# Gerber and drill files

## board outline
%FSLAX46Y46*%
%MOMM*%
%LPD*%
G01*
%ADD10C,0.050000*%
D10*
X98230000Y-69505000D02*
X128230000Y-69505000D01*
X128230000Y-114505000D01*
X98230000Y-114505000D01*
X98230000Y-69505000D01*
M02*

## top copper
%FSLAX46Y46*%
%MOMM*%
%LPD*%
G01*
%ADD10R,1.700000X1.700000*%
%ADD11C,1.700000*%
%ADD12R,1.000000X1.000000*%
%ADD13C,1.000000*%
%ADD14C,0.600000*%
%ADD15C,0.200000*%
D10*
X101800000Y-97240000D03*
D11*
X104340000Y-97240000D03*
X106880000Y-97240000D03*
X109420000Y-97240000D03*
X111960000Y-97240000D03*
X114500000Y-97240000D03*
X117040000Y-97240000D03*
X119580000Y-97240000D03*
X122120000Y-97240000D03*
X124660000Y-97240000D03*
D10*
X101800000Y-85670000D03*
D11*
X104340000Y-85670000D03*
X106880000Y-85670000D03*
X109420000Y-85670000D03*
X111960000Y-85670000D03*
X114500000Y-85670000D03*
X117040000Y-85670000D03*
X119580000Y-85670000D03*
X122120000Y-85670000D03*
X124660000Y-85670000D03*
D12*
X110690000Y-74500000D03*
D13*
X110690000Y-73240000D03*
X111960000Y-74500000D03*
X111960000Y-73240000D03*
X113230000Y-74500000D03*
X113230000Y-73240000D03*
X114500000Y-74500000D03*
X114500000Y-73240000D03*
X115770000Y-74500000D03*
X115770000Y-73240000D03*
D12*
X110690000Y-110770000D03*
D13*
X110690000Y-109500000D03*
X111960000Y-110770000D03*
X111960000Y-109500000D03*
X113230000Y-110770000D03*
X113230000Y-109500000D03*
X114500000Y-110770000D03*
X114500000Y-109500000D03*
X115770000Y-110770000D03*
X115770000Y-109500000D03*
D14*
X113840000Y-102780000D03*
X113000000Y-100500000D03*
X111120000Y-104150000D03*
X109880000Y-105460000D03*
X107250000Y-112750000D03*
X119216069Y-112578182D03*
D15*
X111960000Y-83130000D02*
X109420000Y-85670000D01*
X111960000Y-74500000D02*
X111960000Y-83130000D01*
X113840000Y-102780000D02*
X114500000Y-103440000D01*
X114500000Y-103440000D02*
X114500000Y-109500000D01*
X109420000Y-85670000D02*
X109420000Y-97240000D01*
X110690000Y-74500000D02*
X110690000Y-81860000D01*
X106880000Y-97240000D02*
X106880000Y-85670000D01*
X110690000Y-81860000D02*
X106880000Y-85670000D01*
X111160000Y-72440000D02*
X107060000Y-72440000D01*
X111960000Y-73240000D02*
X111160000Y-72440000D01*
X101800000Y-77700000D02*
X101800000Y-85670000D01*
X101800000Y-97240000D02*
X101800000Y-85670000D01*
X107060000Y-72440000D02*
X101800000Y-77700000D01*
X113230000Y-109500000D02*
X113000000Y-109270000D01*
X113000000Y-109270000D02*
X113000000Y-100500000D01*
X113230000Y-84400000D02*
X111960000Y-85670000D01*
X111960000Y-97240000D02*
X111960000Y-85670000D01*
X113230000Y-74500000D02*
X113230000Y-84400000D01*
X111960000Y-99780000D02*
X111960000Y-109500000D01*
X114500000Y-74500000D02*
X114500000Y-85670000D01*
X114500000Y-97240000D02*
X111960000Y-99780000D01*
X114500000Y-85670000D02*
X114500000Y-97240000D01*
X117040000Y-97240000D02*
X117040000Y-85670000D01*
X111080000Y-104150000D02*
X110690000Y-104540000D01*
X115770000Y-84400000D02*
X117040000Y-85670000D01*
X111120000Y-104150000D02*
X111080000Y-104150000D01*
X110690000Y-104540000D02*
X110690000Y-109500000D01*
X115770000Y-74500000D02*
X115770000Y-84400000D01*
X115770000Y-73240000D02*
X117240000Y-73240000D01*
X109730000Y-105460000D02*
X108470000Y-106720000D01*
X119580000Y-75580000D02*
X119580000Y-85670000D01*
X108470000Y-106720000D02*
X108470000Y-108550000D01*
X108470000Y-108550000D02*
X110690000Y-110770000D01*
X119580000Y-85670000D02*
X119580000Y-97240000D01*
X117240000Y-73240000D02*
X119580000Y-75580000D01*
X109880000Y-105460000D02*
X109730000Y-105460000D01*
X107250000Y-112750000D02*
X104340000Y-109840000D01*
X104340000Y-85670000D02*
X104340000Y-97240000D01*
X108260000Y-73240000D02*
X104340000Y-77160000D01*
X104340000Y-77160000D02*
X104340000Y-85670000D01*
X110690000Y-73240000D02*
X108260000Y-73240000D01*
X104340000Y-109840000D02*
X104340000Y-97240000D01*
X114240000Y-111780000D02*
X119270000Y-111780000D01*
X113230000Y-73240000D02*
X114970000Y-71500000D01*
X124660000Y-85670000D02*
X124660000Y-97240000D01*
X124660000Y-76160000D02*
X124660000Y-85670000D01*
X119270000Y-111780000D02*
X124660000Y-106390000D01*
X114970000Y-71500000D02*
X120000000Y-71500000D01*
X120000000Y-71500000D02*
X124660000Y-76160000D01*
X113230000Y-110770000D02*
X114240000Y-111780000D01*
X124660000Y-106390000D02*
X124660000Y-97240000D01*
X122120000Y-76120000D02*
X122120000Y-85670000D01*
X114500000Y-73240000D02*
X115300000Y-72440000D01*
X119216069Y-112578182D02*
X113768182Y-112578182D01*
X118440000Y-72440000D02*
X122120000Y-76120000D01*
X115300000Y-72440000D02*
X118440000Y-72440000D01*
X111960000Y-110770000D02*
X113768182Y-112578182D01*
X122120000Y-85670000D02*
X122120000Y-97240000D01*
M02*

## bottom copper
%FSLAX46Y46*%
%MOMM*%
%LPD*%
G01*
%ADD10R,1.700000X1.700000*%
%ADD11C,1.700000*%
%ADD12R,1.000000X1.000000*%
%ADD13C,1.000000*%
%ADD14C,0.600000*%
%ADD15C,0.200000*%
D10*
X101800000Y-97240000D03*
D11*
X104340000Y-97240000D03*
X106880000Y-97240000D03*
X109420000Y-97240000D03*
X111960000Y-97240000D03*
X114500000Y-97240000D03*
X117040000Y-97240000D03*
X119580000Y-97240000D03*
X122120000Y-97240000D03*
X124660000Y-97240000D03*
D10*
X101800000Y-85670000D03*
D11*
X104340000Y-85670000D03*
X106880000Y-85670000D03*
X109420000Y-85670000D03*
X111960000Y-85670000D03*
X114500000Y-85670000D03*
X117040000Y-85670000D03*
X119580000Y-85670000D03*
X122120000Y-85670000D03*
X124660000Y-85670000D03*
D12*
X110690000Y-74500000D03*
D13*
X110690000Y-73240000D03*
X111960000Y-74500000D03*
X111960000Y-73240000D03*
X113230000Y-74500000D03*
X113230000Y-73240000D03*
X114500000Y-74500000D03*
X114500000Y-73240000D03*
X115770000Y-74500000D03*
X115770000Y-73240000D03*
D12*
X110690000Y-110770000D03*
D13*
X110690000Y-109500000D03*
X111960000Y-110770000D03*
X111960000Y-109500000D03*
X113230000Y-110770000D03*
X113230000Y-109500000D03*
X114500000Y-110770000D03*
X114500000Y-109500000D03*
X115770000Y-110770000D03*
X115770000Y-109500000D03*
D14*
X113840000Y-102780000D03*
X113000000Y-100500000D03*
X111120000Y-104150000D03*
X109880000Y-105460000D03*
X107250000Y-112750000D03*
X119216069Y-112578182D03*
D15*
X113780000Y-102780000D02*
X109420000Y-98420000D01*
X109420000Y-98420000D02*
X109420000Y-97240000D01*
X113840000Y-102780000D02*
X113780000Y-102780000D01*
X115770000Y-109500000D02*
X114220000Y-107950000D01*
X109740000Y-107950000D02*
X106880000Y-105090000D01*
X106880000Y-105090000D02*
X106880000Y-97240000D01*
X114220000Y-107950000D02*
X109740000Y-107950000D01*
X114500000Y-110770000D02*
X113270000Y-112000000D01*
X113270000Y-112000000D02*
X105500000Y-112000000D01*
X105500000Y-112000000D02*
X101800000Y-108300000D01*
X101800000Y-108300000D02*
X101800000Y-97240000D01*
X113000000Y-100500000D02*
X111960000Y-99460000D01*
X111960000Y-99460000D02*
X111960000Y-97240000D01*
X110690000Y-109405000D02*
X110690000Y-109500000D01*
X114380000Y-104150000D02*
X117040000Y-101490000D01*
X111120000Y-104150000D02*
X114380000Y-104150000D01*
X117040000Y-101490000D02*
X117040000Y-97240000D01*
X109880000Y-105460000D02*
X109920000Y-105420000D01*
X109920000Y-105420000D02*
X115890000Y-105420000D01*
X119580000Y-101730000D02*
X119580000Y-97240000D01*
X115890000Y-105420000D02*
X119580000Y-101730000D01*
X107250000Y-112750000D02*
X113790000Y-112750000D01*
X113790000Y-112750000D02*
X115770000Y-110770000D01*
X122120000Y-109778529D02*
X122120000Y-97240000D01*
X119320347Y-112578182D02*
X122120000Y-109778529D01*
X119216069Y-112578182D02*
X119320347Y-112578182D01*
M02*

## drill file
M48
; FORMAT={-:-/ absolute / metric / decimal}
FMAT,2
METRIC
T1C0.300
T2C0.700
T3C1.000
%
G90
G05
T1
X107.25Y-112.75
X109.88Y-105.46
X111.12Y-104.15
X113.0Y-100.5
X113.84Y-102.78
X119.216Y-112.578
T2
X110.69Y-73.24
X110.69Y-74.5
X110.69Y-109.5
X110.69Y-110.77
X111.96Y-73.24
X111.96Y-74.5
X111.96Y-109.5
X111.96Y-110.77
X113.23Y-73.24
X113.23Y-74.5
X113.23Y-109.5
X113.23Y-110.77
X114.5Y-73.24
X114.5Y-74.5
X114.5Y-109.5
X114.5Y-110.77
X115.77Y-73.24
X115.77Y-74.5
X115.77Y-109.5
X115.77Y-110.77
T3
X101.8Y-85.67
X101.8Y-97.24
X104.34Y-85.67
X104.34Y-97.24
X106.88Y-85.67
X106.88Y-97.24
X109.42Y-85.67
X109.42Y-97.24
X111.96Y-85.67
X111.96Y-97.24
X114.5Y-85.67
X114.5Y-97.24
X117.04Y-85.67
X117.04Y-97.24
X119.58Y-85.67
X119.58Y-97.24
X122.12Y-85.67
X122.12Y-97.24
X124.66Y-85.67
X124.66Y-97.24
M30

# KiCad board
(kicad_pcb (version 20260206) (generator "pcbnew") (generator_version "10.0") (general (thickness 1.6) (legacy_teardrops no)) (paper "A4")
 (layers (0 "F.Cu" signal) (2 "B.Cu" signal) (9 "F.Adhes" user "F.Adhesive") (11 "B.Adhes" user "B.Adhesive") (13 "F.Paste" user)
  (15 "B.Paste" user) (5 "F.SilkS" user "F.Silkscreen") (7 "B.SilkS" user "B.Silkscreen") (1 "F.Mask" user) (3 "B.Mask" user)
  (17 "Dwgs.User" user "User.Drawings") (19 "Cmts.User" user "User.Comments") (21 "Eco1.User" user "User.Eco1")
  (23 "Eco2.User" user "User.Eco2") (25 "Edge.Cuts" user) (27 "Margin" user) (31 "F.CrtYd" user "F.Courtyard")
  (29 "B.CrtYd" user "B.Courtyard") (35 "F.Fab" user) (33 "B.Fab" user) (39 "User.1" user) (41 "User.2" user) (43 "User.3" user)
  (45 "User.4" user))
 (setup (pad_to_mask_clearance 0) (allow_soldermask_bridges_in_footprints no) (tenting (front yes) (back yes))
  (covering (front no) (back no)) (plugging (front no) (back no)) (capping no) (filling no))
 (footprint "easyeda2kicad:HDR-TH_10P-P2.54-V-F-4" (layer "F.Cu") (at 113.23 97.24)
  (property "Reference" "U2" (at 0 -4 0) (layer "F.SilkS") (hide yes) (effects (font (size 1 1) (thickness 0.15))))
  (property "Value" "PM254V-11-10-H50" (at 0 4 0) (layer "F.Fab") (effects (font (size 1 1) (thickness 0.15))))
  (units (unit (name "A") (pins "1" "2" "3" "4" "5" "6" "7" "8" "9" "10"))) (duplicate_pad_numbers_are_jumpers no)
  (pad "1" thru_hole rect (at -11.43 0) (size 1.7 1.7) (drill 0.999998) (layers "*.Cu" "*.Mask") (remove_unused_layers no) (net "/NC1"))
  (pad "2" thru_hole circle (at -8.89 0) (size 1.7 1.7) (drill 0.999998) (layers "*.Cu" "*.Mask") (remove_unused_layers no) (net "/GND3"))
  (pad "3" thru_hole circle (at -6.35 0) (size 1.7 1.7) (drill 0.999998) (layers "*.Cu" "*.Mask") (remove_unused_layers no) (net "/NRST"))
  (pad "4" thru_hole circle (at -3.81 0) (size 1.7 1.7) (drill 0.999998) (layers "*.Cu" "*.Mask") (remove_unused_layers no) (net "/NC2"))
  (pad "5" thru_hole circle (at -1.27 0) (size 1.7 1.7) (drill 0.999998) (layers "*.Cu" "*.Mask") (remove_unused_layers no)
   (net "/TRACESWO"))
  (pad "6" thru_hole circle (at 1.27 0) (size 1.7 1.7) (drill 0.999998) (layers "*.Cu" "*.Mask") (remove_unused_layers no) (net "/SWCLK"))
  (pad "7" thru_hole circle (at 3.81 0) (size 1.7 1.7) (drill 0.999998) (layers "*.Cu" "*.Mask") (remove_unused_layers no) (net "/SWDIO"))
  (pad "8" thru_hole circle (at 6.35 0) (size 1.7 1.7) (drill 0.999998) (layers "*.Cu" "*.Mask") (remove_unused_layers no) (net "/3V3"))
  (pad "9" thru_hole circle (at 8.89 0) (size 1.7 1.7) (drill 0.999998) (layers "*.Cu" "*.Mask") (remove_unused_layers no) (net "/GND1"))
  (pad "10" thru_hole circle (at 11.43 0) (size 1.7 1.7) (drill 0.999998) (layers "*.Cu" "*.Mask") (remove_unused_layers no) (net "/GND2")))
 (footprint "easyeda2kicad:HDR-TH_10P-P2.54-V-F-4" (layer "F.Cu") (at 113.23 85.67)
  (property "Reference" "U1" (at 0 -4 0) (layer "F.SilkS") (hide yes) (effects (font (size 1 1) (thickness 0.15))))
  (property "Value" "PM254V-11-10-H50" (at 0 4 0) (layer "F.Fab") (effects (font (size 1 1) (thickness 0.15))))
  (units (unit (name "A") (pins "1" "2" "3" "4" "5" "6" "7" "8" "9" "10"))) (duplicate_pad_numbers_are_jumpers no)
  (pad "1" thru_hole rect (at -11.43 0) (size 1.7 1.7) (drill 0.999998) (layers "*.Cu" "*.Mask") (remove_unused_layers no) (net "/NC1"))
  (pad "2" thru_hole circle (at -8.89 0) (size 1.7 1.7) (drill 0.999998) (layers "*.Cu" "*.Mask") (remove_unused_layers no) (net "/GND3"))
  (pad "3" thru_hole circle (at -6.35 0) (size 1.7 1.7) (drill 0.999998) (layers "*.Cu" "*.Mask") (remove_unused_layers no) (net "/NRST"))
  (pad "4" thru_hole circle (at -3.81 0) (size 1.7 1.7) (drill 0.999998) (layers "*.Cu" "*.Mask") (remove_unused_layers no) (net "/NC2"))
  (pad "5" thru_hole circle (at -1.27 0) (size 1.7 1.7) (drill 0.999998) (layers "*.Cu" "*.Mask") (remove_unused_layers no)
   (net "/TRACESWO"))
  (pad "6" thru_hole circle (at 1.27 0) (size 1.7 1.7) (drill 0.999998) (layers "*.Cu" "*.Mask") (remove_unused_layers no) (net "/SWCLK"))
  (pad "7" thru_hole circle (at 3.81 0) (size 1.7 1.7) (drill 0.999998) (layers "*.Cu" "*.Mask") (remove_unused_layers no) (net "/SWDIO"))
  (pad "8" thru_hole circle (at 6.35 0) (size 1.7 1.7) (drill 0.999998) (layers "*.Cu" "*.Mask") (remove_unused_layers no) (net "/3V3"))
  (pad "9" thru_hole circle (at 8.89 0) (size 1.7 1.7) (drill 0.999998) (layers "*.Cu" "*.Mask") (remove_unused_layers no) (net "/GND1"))
  (pad "10" thru_hole circle (at 11.43 0) (size 1.7 1.7) (drill 0.999998) (layers "*.Cu" "*.Mask") (remove_unused_layers no) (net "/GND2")))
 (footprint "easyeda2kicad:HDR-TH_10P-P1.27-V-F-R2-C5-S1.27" (layer "F.Cu") (at 113.23 73.87)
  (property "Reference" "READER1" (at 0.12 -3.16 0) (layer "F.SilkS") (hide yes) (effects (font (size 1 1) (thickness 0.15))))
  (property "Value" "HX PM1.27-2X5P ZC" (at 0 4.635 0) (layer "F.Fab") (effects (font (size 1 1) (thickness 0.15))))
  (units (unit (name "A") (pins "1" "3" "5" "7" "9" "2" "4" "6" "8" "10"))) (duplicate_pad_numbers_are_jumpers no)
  (pad "1" thru_hole rect (at -2.54 0.63) (size 1 1) (drill 0.700024) (layers "*.Cu" "*.Mask") (remove_unused_layers no) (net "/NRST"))
  (pad "2" thru_hole circle (at -2.54 -0.63) (size 1 1) (drill 0.700024) (layers "*.Cu" "*.Mask") (remove_unused_layers no) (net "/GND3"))
  (pad "3" thru_hole circle (at -1.27 0.63) (size 1 1) (drill 0.700024) (layers "*.Cu" "*.Mask") (remove_unused_layers no) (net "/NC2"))
  (pad "4" thru_hole circle (at -1.27 -0.63) (size 1 1) (drill 0.700024) (layers "*.Cu" "*.Mask") (remove_unused_layers no) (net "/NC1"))
  (pad "5" thru_hole circle (at 0 0.63) (size 1 1) (drill 0.700024) (layers "*.Cu" "*.Mask") (remove_unused_layers no) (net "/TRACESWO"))
  (pad "6" thru_hole circle (at 0 -0.63) (size 1 1) (drill 0.700024) (layers "*.Cu" "*.Mask") (remove_unused_layers no) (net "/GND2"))
  (pad "7" thru_hole circle (at 1.27 0.63) (size 1 1) (drill 0.700024) (layers "*.Cu" "*.Mask") (remove_unused_layers no) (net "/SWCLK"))
  (pad "8" thru_hole circle (at 1.27 -0.63) (size 1 1) (drill 0.700024) (layers "*.Cu" "*.Mask") (remove_unused_layers no) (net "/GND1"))
  (pad "9" thru_hole circle (at 2.54 0.63) (size 1 1) (drill 0.700024) (layers "*.Cu" "*.Mask") (remove_unused_layers no) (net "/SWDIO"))
  (pad "10" thru_hole circle (at 2.54 -0.63) (size 1 1) (drill 0.700024) (layers "*.Cu" "*.Mask") (remove_unused_layers no) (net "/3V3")))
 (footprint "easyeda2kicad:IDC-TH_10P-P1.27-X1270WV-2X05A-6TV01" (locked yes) (layer "F.Cu") (at 113.23 110.14)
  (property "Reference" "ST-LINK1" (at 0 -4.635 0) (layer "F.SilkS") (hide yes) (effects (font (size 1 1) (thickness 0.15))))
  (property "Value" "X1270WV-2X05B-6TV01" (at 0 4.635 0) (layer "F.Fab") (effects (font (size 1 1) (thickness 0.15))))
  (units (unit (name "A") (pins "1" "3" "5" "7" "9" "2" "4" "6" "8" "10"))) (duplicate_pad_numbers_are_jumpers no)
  (pad "1" thru_hole rect (at -2.54 0.63) (size 1 1) (drill 0.700024) (layers "*.Cu" "*.Mask") (remove_unused_layers no) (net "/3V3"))
  (pad "2" thru_hole circle (at -2.54 -0.64) (size 1 1) (drill 0.700024) (layers "*.Cu" "*.Mask") (remove_unused_layers no) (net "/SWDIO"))
  (pad "3" thru_hole circle (at -1.27 0.63) (size 1 1) (drill 0.700024) (layers "*.Cu" "*.Mask") (remove_unused_layers no) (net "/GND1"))
  (pad "4" thru_hole circle (at -1.27 -0.64) (size 1 1) (drill 0.700024) (layers "*.Cu" "*.Mask") (remove_unused_layers no) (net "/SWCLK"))
  (pad "5" thru_hole circle (at 0 0.63) (size 1 1) (drill 0.700024) (layers "*.Cu" "*.Mask") (remove_unused_layers no) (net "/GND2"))
  (pad "6" thru_hole circle (at 0 -0.64) (size 1 1) (drill 0.700024) (layers "*.Cu" "*.Mask") (remove_unused_layers no) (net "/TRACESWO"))
  (pad "7" thru_hole circle (at 1.27 0.63) (size 1 1) (drill 0.700024) (layers "*.Cu" "*.Mask") (remove_unused_layers no) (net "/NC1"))
  (pad "8" thru_hole circle (at 1.27 -0.64) (size 1 1) (drill 0.700024) (layers "*.Cu" "*.Mask") (remove_unused_layers no) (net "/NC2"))
  (pad "9" thru_hole circle (at 2.54 0.63) (size 1 1) (drill 0.700024) (layers "*.Cu" "*.Mask") (remove_unused_layers no) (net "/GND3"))
  (pad "10" thru_hole circle (at 2.54 -0.64) (size 1 1) (drill 0.700024) (layers "*.Cu" "*.Mask") (remove_unused_layers no) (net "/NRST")))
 (gr_rect (start 98.23 69.505) (end 128.23 114.505) (stroke (width 0.05) (type default)) (fill no) (layer "Edge.Cuts"))
 (segment (start 111.96 83.13) (end 109.42 85.67) (width 0.2) (layer "F.Cu") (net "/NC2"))
 (segment (start 111.96 74.5) (end 111.96 83.13) (width 0.2) (layer "F.Cu") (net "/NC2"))
 (segment (start 113.84 102.78) (end 114.5 103.44) (width 0.2) (layer "F.Cu") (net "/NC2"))
 (segment (start 114.5 103.44) (end 114.5 109.5) (width 0.2) (layer "F.Cu") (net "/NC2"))
 (segment (start 109.42 85.67) (end 109.42 97.24) (width 0.2) (layer "F.Cu") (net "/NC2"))
 (via (at 113.84 102.78) (size 0.6) (drill 0.3) (layers "F.Cu" "B.Cu") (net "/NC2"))
 (segment (start 113.78 102.78) (end 109.42 98.42) (width 0.2) (layer "B.Cu") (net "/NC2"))
 (segment (start 109.42 98.42) (end 109.42 97.24) (width 0.2) (layer "B.Cu") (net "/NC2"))
 (segment (start 113.84 102.78) (end 113.78 102.78) (width 0.2) (layer "B.Cu") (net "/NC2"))
 (segment (start 110.69 74.5) (end 110.69 81.86) (width 0.2) (layer "F.Cu") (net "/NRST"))
 (segment (start 106.88 97.24) (end 106.88 85.67) (width 0.2) (layer "F.Cu") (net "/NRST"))
 (segment (start 110.69 81.86) (end 106.88 85.67) (width 0.2) (layer "F.Cu") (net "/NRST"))
 (segment (start 115.77 109.5) (end 114.22 107.95) (width 0.2) (layer "B.Cu") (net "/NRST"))
 (segment (start 109.74 107.95) (end 106.88 105.09) (width 0.2) (layer "B.Cu") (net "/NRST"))
 (segment (start 106.88 105.09) (end 106.88 97.24) (width 0.2) (layer "B.Cu") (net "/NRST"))
 (segment (start 114.22 107.95) (end 109.74 107.95) (width 0.2) (layer "B.Cu") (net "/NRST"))
 (segment (start 111.16 72.44) (end 107.06 72.44) (width 0.2) (layer "F.Cu") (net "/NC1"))
 (segment (start 111.96 73.24) (end 111.16 72.44) (width 0.2) (layer "F.Cu") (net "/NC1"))
 (segment (start 101.8 77.7) (end 101.8 85.67) (width 0.2) (layer "F.Cu") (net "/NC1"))
 (segment (start 101.8 97.24) (end 101.8 85.67) (width 0.2) (layer "F.Cu") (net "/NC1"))
 (segment (start 107.06 72.44) (end 101.8 77.7) (width 0.2) (layer "F.Cu") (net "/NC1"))
 (segment (start 114.5 110.77) (end 113.27 112) (width 0.2) (layer "B.Cu") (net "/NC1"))
 (segment (start 113.27 112) (end 105.5 112) (width 0.2) (layer "B.Cu") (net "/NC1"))
 (segment (start 105.5 112) (end 101.8 108.3) (width 0.2) (layer "B.Cu") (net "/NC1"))
 (segment (start 101.8 108.3) (end 101.8 97.24) (width 0.2) (layer "B.Cu") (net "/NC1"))
 (segment (start 113.23 109.5) (end 113 109.27) (width 0.2) (layer "F.Cu") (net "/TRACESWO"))
 (segment (start 113 109.27) (end 113 100.5) (width 0.2) (layer "F.Cu") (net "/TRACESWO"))
 (segment (start 113.23 84.4) (end 111.96 85.67) (width 0.2) (layer "F.Cu") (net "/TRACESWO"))
 (segment (start 111.96 97.24) (end 111.96 85.67) (width 0.2) (layer "F.Cu") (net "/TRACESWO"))
 (segment (start 113.23 74.5) (end 113.23 84.4) (width 0.2) (layer "F.Cu") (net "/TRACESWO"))
 (via (at 113 100.5) (size 0.6) (drill 0.3) (layers "F.Cu" "B.Cu") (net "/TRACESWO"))
 (segment (start 113 100.5) (end 111.96 99.46) (width 0.2) (layer "B.Cu") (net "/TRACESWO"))
 (segment (start 111.96 99.46) (end 111.96 97.24) (width 0.2) (layer "B.Cu") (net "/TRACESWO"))
 (segment (start 111.96 99.78) (end 111.96 109.5) (width 0.2) (layer "F.Cu") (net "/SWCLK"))
 (segment (start 114.5 74.5) (end 114.5 85.67) (width 0.2) (layer "F.Cu") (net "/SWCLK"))
 (segment (start 114.5 97.24) (end 111.96 99.78) (width 0.2) (layer "F.Cu") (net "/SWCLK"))
 (segment (start 114.5 85.67) (end 114.5 97.24) (width 0.2) (layer "F.Cu") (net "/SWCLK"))
 (segment (start 117.04 97.24) (end 117.04 85.67) (width 0.2) (layer "F.Cu") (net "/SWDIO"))
 (segment (start 111.08 104.15) (end 110.69 104.54) (width 0.2) (layer "F.Cu") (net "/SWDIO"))
 (segment (start 115.77 84.4) (end 117.04 85.67) (width 0.2) (layer "F.Cu") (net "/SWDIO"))
 (segment (start 111.12 104.15) (end 111.08 104.15) (width 0.2) (layer "F.Cu") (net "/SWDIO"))
 (segment (start 110.69 104.54) (end 110.69 109.5) (width 0.2) (layer "F.Cu") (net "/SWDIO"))
 (segment (start 115.77 74.5) (end 115.77 84.4) (width 0.2) (layer "F.Cu") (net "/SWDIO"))
 (via (at 111.12 104.15) (size 0.6) (drill 0.3) (layers "F.Cu" "B.Cu") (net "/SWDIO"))
 (segment (start 110.69 109.405) (end 110.69 109.5) (width 0.2) (layer "B.Cu") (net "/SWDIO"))
 (segment (start 114.38 104.15) (end 117.04 101.49) (width 0.2) (layer "B.Cu") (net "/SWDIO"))
 (segment (start 111.12 104.15) (end 114.38 104.15) (width 0.2) (layer "B.Cu") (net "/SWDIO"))
 (segment (start 117.04 101.49) (end 117.04 97.24) (width 0.2) (layer "B.Cu") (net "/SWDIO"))
 (segment (start 115.77 73.24) (end 117.24 73.24) (width 0.2) (layer "F.Cu") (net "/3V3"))
 (segment (start 109.73 105.46) (end 108.47 106.72) (width 0.2) (layer "F.Cu") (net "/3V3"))
 (segment (start 119.58 75.58) (end 119.58 85.67) (width 0.2) (layer "F.Cu") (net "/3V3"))
 (segment (start 108.47 106.72) (end 108.47 108.55) (width 0.2) (layer "F.Cu") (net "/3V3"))
 (segment (start 108.47 108.55) (end 110.69 110.77) (width 0.2) (layer "F.Cu") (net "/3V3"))
 (segment (start 119.58 85.67) (end 119.58 97.24) (width 0.2) (layer "F.Cu") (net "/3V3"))
 (segment (start 117.24 73.24) (end 119.58 75.58) (width 0.2) (layer "F.Cu") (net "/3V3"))
 (segment (start 109.88 105.46) (end 109.73 105.46) (width 0.2) (layer "F.Cu") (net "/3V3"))
 (via (at 109.88 105.46) (size 0.6) (drill 0.3) (layers "F.Cu" "B.Cu") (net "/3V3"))
 (segment (start 109.88 105.46) (end 109.92 105.42) (width 0.2) (layer "B.Cu") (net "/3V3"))
 (segment (start 109.92 105.42) (end 115.89 105.42) (width 0.2) (layer "B.Cu") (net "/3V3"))
 (segment (start 119.58 101.73) (end 119.58 97.24) (width 0.2) (layer "B.Cu") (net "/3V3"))
 (segment (start 115.89 105.42) (end 119.58 101.73) (width 0.2) (layer "B.Cu") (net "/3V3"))
 (segment (start 107.25 112.75) (end 104.34 109.84) (width 0.2) (layer "F.Cu") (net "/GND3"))
 (segment (start 104.34 85.67) (end 104.34 97.24) (width 0.2) (layer "F.Cu") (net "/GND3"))
 (segment (start 108.26 73.24) (end 104.34 77.16) (width 0.2) (layer "F.Cu") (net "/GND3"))
 (segment (start 104.34 77.16) (end 104.34 85.67) (width 0.2) (layer "F.Cu") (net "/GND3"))
 (segment (start 110.69 73.24) (end 108.26 73.24) (width 0.2) (layer "F.Cu") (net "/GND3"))
 (segment (start 104.34 109.84) (end 104.34 97.24) (width 0.2) (layer "F.Cu") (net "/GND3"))
 (via (at 107.25 112.75) (size 0.6) (drill 0.3) (layers "F.Cu" "B.Cu") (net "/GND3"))
 (segment (start 107.25 112.75) (end 113.79 112.75) (width 0.2) (layer "B.Cu") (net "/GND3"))
 (segment (start 113.79 112.75) (end 115.77 110.77) (width 0.2) (layer "B.Cu") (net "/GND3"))
 (segment (start 114.24 111.78) (end 119.27 111.78) (width 0.2) (layer "F.Cu") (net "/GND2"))
 (segment (start 113.23 73.24) (end 114.97 71.5) (width 0.2) (layer "F.Cu") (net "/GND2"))
 (segment (start 124.66 85.67) (end 124.66 97.24) (width 0.2) (layer "F.Cu") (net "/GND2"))
 (segment (start 124.66 76.16) (end 124.66 85.67) (width 0.2) (layer "F.Cu") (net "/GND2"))
 (segment (start 119.27 111.78) (end 124.66 106.39) (width 0.2) (layer "F.Cu") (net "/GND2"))
 (segment (start 114.97 71.5) (end 120 71.5) (width 0.2) (layer "F.Cu") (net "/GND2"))
 (segment (start 120 71.5) (end 124.66 76.16) (width 0.2) (layer "F.Cu") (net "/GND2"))
 (segment (start 113.23 110.77) (end 114.24 111.78) (width 0.2) (layer "F.Cu") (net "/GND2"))
 (segment (start 124.66 106.39) (end 124.66 97.24) (width 0.2) (layer "F.Cu") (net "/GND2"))
 (segment (start 122.12 76.12) (end 122.12 85.67) (width 0.2) (layer "F.Cu") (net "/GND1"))
 (segment (start 114.5 73.24) (end 115.3 72.44) (width 0.2) (layer "F.Cu") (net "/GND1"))
 (segment (start 119.216069 112.578182) (end 113.768182 112.578182) (width 0.2) (layer "F.Cu") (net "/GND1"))
 (segment (start 118.44 72.44) (end 122.12 76.12) (width 0.2) (layer "F.Cu") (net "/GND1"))
 (segment (start 115.3 72.44) (end 118.44 72.44) (width 0.2) (layer "F.Cu") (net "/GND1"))
 (segment (start 111.96 110.77) (end 113.768182 112.578182) (width 0.2) (layer "F.Cu") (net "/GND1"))
 (segment (start 122.12 85.67) (end 122.12 97.24) (width 0.2) (layer "F.Cu") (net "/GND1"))
 (via (at 119.216069 112.578182) (size 0.6) (drill 0.3) (layers "F.Cu" "B.Cu") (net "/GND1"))
 (segment (start 122.12 109.778529) (end 122.12 97.24) (width 0.2) (layer "B.Cu") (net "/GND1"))
 (segment (start 119.320347 112.578182) (end 122.12 109.778529) (width 0.2) (layer "B.Cu") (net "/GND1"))
 (segment (start 119.216069 112.578182) (end 119.320347 112.578182) (width 0.2) (layer "B.Cu") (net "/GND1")))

